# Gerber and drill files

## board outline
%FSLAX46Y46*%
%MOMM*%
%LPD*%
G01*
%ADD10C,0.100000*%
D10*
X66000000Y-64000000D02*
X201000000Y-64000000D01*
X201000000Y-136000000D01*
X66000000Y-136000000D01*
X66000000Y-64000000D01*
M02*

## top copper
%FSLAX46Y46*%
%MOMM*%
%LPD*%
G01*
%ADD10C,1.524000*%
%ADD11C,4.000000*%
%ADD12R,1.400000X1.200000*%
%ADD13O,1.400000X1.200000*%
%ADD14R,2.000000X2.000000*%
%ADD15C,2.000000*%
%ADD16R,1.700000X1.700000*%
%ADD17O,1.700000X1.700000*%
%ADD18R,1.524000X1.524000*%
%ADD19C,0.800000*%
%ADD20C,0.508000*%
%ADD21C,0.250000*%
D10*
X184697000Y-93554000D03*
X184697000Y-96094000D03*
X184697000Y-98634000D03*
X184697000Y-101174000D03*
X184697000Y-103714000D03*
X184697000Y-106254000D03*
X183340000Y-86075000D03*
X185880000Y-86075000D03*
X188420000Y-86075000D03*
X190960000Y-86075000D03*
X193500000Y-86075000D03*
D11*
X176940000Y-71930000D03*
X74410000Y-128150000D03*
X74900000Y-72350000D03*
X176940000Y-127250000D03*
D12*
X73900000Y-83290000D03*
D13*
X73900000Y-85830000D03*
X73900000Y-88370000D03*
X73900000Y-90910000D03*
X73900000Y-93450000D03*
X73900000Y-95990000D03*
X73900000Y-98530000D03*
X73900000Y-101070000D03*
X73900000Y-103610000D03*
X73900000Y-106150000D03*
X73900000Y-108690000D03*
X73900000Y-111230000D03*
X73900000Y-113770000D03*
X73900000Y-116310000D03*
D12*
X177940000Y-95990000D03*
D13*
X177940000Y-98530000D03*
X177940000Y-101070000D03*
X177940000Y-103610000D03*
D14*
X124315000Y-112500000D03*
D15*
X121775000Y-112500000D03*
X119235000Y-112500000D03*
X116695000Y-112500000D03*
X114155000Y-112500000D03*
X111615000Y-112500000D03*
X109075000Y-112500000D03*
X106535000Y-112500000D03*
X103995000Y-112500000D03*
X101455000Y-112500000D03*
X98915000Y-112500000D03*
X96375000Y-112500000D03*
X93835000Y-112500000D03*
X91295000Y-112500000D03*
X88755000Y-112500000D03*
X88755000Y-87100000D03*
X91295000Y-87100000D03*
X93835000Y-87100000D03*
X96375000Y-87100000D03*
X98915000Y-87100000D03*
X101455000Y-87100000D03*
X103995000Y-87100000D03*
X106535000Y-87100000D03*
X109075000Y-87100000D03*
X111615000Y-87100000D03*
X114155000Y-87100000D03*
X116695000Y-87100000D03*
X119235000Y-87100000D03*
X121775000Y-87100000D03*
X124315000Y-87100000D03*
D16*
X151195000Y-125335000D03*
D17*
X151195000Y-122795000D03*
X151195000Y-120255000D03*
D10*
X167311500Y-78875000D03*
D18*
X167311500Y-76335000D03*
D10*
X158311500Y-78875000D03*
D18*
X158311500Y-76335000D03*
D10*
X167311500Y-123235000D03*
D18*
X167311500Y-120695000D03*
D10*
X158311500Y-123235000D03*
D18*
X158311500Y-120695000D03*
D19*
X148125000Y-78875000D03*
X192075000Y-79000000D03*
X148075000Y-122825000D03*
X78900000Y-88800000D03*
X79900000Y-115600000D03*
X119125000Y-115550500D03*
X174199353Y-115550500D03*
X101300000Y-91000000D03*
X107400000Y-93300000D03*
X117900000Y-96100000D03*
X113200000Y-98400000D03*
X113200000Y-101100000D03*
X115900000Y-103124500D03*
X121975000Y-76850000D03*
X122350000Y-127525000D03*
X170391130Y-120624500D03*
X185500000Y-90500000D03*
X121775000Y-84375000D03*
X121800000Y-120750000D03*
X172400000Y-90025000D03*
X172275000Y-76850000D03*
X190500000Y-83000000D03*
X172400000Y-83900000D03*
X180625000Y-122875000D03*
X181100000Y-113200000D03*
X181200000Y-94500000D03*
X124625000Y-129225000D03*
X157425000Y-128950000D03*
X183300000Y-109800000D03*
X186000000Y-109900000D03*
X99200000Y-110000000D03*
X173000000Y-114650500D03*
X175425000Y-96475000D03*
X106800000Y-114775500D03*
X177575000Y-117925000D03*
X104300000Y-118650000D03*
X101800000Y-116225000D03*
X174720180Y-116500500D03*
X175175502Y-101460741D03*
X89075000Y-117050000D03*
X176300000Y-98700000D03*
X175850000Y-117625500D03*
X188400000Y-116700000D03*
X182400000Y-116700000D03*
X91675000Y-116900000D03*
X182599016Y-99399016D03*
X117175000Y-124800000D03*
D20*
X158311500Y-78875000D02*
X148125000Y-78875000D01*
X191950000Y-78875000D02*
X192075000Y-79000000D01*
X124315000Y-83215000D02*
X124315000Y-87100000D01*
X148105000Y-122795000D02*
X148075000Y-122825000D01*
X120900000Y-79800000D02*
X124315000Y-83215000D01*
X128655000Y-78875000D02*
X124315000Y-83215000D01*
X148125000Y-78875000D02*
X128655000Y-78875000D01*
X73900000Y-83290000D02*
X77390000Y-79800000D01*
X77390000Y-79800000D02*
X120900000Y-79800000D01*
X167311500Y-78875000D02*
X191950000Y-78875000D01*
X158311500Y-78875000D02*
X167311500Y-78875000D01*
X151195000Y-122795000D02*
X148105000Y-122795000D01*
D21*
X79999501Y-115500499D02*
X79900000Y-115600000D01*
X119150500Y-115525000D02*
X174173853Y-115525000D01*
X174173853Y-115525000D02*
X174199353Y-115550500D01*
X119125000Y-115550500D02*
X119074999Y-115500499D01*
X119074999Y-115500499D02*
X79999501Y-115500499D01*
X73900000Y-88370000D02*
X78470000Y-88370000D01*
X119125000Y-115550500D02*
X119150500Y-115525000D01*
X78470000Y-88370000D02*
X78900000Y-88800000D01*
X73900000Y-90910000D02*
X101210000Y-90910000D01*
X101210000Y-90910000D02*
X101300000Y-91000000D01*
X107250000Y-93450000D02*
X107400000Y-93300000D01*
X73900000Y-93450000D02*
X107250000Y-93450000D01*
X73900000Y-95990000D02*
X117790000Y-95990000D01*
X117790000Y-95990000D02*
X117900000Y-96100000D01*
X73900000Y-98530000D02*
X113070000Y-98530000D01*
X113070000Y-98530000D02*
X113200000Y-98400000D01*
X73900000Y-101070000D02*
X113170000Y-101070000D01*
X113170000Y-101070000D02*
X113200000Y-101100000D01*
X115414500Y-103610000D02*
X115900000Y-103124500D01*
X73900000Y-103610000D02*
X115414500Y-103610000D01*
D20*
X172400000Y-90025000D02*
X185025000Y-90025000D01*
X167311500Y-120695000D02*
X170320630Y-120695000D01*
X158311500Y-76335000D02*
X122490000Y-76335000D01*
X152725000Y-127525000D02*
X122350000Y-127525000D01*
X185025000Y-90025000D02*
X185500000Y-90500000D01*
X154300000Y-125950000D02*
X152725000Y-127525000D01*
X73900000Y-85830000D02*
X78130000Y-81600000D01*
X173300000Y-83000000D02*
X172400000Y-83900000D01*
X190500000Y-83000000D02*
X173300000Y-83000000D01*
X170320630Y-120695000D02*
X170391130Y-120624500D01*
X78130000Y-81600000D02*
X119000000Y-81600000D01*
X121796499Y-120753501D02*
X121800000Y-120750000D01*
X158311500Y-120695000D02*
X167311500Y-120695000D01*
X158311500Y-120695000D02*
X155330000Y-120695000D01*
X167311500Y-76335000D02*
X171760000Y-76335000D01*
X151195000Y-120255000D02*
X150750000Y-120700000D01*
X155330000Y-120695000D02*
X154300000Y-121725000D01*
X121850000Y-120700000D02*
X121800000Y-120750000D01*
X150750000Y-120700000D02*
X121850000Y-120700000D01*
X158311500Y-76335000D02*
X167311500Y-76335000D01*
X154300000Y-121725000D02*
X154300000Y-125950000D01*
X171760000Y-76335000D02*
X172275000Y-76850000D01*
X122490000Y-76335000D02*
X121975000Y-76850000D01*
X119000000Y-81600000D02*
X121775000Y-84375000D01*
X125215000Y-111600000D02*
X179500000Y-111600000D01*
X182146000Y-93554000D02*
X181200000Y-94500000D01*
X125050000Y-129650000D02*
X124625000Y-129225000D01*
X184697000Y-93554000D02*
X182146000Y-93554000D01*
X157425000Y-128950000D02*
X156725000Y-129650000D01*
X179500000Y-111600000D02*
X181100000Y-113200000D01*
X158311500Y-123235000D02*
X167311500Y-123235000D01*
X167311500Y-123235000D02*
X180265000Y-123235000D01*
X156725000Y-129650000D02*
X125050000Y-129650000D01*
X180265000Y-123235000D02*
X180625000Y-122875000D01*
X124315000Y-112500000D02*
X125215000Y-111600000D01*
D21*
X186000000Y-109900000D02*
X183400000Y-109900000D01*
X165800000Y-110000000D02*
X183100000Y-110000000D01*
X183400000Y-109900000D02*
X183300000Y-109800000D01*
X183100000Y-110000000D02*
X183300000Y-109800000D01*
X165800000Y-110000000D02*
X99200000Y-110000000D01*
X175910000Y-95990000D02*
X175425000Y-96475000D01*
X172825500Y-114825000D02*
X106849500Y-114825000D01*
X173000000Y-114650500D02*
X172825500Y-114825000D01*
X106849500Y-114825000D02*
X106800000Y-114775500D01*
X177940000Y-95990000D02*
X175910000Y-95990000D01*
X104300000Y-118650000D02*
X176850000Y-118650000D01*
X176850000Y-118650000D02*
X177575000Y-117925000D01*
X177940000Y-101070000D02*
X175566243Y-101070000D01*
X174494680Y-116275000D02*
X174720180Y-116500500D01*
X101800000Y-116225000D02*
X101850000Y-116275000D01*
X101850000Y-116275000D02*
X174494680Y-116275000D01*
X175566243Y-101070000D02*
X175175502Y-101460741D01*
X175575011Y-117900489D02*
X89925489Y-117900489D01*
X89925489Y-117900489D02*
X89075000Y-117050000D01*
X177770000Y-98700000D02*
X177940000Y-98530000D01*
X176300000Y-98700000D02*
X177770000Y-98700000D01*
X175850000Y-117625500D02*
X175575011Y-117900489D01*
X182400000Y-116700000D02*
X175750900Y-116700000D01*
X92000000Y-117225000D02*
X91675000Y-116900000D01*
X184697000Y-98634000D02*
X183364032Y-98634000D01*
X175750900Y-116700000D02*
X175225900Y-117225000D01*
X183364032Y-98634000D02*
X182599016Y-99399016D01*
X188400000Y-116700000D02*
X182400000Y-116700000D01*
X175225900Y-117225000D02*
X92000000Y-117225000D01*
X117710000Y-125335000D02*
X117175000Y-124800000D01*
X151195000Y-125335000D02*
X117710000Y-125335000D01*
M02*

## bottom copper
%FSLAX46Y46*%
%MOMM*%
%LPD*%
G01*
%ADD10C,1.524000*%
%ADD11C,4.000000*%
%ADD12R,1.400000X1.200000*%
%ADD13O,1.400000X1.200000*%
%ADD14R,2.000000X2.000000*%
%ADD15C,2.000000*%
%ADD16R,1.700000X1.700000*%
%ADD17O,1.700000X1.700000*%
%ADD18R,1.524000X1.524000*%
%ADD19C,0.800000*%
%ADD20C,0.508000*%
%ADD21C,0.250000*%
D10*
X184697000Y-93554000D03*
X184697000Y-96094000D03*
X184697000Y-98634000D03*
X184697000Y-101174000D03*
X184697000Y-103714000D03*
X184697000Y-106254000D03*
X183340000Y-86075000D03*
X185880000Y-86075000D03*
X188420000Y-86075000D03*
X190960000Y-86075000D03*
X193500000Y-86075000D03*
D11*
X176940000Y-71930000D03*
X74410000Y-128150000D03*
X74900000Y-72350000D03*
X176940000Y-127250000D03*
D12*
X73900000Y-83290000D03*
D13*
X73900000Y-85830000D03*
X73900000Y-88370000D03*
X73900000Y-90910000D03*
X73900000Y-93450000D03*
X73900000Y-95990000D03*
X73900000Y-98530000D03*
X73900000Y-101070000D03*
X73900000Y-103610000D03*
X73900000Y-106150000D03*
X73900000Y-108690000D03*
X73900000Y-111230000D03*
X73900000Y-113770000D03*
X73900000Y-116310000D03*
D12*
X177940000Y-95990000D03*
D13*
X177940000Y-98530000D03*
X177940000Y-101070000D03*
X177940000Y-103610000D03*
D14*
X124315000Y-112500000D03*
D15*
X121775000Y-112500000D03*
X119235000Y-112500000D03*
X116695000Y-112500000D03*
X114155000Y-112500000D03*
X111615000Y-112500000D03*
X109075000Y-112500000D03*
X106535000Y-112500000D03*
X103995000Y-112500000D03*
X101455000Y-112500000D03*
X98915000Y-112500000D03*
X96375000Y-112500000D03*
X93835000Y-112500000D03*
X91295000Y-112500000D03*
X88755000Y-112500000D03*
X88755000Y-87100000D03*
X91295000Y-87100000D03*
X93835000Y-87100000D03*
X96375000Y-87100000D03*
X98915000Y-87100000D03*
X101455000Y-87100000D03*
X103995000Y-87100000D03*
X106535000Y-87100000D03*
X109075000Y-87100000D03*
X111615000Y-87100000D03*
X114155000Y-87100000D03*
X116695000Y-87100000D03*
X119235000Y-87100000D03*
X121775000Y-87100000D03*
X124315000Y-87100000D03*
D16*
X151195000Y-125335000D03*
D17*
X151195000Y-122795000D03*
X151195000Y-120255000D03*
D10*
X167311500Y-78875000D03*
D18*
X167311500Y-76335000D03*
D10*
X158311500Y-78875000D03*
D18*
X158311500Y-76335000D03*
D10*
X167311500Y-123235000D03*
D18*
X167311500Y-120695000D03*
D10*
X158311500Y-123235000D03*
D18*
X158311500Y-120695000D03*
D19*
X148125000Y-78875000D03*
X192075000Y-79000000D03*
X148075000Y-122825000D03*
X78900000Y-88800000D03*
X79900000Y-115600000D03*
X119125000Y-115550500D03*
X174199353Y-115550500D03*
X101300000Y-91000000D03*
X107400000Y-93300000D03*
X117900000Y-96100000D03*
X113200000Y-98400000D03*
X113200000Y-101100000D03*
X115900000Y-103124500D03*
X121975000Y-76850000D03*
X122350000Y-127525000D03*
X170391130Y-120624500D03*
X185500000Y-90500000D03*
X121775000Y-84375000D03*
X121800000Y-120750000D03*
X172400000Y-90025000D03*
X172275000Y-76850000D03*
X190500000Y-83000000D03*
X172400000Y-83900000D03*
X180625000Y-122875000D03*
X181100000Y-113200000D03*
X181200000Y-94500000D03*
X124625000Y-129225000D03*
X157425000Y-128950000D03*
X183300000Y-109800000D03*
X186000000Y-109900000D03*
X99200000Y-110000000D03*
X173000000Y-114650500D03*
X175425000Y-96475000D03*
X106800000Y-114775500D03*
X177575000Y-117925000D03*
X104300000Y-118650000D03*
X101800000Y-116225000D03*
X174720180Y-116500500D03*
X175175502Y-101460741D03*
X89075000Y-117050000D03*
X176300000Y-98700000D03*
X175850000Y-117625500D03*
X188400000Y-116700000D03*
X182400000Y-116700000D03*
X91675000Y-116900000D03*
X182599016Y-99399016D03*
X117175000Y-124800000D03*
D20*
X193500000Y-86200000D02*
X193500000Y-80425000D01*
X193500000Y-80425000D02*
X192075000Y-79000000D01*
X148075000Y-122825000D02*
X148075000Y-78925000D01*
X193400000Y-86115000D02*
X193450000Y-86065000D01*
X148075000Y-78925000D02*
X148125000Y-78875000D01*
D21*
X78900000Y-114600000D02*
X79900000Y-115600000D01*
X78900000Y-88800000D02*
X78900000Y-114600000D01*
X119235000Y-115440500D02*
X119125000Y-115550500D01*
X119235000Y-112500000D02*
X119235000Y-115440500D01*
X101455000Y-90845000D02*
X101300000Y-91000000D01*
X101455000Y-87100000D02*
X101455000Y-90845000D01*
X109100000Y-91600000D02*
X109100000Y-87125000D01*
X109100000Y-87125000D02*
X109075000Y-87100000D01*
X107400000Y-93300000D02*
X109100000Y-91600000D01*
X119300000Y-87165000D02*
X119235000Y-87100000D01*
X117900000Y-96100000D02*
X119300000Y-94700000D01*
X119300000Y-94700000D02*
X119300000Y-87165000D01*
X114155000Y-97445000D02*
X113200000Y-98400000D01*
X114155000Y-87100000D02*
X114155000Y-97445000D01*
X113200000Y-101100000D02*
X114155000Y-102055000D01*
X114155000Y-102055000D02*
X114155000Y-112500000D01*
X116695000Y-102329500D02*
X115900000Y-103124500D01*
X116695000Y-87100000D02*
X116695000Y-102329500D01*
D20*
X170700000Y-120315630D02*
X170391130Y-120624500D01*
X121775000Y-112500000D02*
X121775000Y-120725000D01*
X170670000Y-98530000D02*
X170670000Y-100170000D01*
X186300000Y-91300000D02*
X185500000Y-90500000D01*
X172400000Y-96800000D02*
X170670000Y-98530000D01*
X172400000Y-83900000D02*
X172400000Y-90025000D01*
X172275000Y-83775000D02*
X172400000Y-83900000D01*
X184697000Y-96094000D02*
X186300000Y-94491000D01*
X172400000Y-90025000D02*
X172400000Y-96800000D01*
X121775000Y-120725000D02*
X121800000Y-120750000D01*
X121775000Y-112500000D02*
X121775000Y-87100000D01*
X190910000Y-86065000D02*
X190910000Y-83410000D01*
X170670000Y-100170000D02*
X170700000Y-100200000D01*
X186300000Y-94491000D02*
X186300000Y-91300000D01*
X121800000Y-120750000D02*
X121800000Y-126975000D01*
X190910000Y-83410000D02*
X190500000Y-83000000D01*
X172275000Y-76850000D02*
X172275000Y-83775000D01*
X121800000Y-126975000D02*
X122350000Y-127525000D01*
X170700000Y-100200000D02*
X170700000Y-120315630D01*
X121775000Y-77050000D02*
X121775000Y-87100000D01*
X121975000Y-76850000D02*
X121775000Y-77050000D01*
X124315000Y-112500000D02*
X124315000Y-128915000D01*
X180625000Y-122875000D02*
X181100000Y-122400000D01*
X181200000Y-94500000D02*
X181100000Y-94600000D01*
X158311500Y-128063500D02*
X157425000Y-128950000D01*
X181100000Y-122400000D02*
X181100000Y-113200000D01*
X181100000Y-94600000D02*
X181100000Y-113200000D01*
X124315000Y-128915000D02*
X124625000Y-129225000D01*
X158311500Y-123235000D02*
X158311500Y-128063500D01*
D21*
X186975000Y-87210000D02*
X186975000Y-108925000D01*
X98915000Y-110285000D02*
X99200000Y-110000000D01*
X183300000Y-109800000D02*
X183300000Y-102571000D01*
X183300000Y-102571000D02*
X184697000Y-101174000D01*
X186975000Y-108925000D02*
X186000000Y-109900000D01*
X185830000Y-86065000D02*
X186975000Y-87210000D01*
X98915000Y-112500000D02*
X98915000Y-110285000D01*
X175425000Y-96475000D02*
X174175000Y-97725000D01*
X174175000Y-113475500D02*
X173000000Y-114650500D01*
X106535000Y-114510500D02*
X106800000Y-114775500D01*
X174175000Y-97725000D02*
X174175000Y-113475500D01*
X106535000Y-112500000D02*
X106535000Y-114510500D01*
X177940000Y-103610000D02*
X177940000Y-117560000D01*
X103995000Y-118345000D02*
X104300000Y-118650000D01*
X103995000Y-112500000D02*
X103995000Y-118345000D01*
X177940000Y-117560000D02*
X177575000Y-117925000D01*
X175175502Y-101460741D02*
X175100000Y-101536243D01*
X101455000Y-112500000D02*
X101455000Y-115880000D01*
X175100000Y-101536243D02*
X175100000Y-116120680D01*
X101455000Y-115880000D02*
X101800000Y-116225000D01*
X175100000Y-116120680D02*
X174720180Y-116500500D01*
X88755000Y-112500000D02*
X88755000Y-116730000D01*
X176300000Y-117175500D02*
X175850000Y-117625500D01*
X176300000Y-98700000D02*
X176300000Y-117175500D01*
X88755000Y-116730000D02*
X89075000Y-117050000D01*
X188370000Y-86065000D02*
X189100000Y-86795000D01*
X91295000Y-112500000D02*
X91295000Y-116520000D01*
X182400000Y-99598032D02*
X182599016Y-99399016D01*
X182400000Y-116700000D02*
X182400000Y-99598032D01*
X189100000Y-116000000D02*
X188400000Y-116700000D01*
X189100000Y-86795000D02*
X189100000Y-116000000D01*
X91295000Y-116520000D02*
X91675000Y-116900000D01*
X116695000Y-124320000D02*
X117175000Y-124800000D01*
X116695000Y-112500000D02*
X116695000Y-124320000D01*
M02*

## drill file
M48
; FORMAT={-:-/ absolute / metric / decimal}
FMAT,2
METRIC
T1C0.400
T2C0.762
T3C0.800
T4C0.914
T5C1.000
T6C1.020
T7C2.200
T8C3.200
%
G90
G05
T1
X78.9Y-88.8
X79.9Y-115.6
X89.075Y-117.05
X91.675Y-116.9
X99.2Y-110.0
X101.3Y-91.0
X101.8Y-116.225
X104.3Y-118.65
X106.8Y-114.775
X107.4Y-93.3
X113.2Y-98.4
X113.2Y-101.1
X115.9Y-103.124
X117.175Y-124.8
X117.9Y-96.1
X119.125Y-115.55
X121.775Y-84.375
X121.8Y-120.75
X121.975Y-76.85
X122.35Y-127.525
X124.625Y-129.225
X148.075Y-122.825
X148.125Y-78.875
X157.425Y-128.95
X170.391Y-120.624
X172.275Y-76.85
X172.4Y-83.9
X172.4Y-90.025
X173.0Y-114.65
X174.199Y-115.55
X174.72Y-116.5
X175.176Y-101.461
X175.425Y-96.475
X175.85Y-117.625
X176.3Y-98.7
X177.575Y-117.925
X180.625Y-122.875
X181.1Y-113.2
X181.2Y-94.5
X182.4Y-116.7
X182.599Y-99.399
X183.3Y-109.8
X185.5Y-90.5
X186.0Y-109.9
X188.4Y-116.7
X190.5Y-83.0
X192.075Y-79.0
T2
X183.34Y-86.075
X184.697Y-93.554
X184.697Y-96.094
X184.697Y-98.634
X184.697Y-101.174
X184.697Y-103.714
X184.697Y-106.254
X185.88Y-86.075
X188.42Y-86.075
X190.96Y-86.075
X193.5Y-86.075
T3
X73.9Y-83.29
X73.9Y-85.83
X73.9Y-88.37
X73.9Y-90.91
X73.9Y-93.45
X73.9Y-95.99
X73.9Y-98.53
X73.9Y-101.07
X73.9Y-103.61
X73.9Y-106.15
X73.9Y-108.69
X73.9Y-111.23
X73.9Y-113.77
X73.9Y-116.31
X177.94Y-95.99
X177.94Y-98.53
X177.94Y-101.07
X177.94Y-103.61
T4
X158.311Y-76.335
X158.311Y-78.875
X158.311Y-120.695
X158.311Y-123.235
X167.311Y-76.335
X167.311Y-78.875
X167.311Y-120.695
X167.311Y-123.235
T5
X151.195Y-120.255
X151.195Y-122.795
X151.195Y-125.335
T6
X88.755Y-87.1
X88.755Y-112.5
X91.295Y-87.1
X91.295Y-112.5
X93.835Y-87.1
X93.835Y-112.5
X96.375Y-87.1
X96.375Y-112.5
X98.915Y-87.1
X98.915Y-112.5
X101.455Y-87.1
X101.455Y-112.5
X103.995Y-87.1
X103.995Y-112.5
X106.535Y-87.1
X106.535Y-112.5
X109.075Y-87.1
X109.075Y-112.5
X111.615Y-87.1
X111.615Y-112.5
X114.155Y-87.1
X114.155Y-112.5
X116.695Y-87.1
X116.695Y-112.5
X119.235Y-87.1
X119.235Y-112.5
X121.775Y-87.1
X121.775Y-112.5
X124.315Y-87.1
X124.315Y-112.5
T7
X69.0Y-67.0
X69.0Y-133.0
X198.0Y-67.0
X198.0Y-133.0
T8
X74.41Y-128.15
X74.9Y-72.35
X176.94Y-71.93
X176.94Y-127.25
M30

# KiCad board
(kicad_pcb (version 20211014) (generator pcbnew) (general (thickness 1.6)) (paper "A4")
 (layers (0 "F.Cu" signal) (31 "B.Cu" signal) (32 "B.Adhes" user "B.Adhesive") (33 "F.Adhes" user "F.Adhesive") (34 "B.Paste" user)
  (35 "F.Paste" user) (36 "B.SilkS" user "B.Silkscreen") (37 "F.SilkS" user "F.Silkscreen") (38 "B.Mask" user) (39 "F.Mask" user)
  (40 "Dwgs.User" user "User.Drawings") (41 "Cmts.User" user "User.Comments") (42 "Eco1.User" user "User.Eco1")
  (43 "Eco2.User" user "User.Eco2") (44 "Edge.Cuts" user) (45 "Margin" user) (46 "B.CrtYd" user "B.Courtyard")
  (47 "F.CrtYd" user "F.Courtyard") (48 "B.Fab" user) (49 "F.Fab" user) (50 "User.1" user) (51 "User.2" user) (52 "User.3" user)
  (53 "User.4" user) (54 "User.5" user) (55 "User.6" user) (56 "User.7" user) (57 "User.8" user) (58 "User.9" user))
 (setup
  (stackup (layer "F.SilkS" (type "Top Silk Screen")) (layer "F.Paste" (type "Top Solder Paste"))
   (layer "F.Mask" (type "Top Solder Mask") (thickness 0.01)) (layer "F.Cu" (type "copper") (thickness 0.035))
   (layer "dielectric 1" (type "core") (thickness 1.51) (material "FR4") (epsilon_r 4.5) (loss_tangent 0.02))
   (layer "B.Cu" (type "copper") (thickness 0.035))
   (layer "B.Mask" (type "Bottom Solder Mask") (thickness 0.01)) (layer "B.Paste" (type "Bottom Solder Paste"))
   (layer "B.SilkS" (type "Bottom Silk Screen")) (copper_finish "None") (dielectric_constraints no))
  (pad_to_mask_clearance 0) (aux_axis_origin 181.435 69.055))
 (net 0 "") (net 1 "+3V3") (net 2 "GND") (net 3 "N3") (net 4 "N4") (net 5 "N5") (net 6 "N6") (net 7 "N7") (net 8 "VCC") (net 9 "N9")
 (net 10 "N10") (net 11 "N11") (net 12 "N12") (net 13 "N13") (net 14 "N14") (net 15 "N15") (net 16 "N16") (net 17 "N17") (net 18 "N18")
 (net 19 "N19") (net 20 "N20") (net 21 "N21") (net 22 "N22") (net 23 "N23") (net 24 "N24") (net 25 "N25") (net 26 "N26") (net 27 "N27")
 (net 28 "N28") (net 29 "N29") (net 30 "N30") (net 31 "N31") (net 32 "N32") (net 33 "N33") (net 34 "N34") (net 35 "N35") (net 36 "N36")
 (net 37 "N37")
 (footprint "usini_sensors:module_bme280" (layer "F.Cu") (at 189.777 106)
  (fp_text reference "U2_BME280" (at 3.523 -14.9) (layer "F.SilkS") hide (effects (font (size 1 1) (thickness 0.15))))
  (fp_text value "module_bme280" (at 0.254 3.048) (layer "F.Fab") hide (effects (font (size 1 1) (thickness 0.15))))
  (pad "1" thru_hole circle locked (at -5.08 -12.446) (size 1.524 1.524) (drill 0.762) (layers *.Cu *.Mask) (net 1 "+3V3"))
  (pad "2" thru_hole circle locked (at -5.08 -9.906) (size 1.524 1.524) (drill 0.762) (layers *.Cu *.Mask) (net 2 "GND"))
  (pad "3" thru_hole circle locked (at -5.08 -7.366) (size 1.524 1.524) (drill 0.762) (layers *.Cu *.Mask) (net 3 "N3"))
  (pad "4" thru_hole circle locked (at -5.08 -4.826) (size 1.524 1.524) (drill 0.762) (layers *.Cu *.Mask) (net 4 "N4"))
  (pad "5" thru_hole circle locked (at -5.08 -2.286) (size 1.524 1.524) (drill 0.762) (layers *.Cu *.Mask) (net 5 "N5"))
  (pad "6" thru_hole circle locked (at -5.08 0.254) (size 1.524 1.524) (drill 0.762) (layers *.Cu *.Mask) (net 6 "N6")))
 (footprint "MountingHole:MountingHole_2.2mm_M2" (layer "F.Cu") (at 69 67)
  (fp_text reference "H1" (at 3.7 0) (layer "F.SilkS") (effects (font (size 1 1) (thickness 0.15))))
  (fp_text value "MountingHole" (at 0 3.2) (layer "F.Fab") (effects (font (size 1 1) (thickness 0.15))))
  (pad "" np_thru_hole circle locked (at 0 0) (size 2.2 2.2) (drill 2.2) (layers *.Cu *.Mask)))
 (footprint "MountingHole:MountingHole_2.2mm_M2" (layer "F.Cu") (at 198 67)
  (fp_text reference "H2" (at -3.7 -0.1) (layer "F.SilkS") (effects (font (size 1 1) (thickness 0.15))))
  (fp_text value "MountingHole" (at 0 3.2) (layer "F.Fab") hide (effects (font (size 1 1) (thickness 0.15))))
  (pad "" np_thru_hole circle locked (at 0 0) (size 2.2 2.2) (drill 2.2) (layers *.Cu *.Mask)))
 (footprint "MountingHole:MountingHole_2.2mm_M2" (layer "F.Cu") (at 198 133)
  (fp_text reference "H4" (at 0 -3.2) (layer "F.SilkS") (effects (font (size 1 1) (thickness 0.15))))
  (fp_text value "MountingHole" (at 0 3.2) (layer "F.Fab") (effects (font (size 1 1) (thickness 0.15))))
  (pad "" np_thru_hole circle locked (at 0 0) (size 2.2 2.2) (drill 2.2) (layers *.Cu *.Mask)))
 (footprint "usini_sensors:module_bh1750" (layer "F.Cu") (at 193.5 86.075 90)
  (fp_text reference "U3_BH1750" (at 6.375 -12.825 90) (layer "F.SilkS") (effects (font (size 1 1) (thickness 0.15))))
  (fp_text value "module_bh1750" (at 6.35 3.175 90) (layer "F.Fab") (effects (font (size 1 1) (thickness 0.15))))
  (pad "1" thru_hole circle locked (at 0 -10.16 90) (size 1.524 1.524) (drill 0.762) (layers *.Cu *.Mask) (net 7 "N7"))
  (pad "2" thru_hole circle locked (at 0 -7.62 90) (size 1.524 1.524) (drill 0.762) (layers *.Cu *.Mask) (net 4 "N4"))
  (pad "3" thru_hole circle locked (at 0 -5.08 90) (size 1.524 1.524) (drill 0.762) (layers *.Cu *.Mask) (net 3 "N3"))
  (pad "4" thru_hole circle locked (at 0 -2.54 90) (size 1.524 1.524) (drill 0.762) (layers *.Cu *.Mask) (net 2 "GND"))
  (pad "5" thru_hole circle locked (at 0 0 90) (size 1.524 1.524) (drill 0.762) (layers *.Cu *.Mask) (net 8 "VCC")))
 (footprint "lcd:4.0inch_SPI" (layer "F.Cu") (at 71.9 68.93)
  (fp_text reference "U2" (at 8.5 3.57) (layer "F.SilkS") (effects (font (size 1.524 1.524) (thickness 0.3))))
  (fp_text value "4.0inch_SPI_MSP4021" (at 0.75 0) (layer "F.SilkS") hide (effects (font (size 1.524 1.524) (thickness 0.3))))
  (pad "" np_thru_hole circle (at 105.04 3 270) (size 4 4) (drill 3.2) (layers F&B.Cu *.Mask))
  (pad "" np_thru_hole circle (at 2.51 59.22 270) (size 4 4) (drill 3.2) (layers F&B.Cu *.Mask))
  (pad "" np_thru_hole circle (at 3 3.42 270) (size 4 4) (drill 3.2) (layers F&B.Cu *.Mask))
  (pad "" np_thru_hole circle (at 105.04 58.32 270) (size 4 4) (drill 3.2) (layers F&B.Cu *.Mask))
  (pad "1" thru_hole rect (at 2 14.36 270) (size 1.2 1.4) (drill 0.8) (layers *.Cu *.Mask) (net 8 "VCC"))
  (pad "2" thru_hole oval (at 2 16.9 270) (size 1.2 1.4) (drill 0.8) (layers *.Cu *.Mask) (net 2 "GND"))
  (pad "3" thru_hole oval (at 2 19.44 270) (size 1.2 1.4) (drill 0.8) (layers *.Cu *.Mask) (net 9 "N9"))
  (pad "4" thru_hole oval (at 2 21.98 270) (size 1.2 1.4) (drill 0.8) (layers *.Cu *.Mask) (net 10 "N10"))
  (pad "5" thru_hole oval (at 2 24.52 270) (size 1.2 1.4) (drill 0.8) (layers *.Cu *.Mask) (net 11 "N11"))
  (pad "6" thru_hole oval (at 2 27.06 270) (size 1.2 1.4) (drill 0.8) (layers *.Cu *.Mask) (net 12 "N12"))
  (pad "7" thru_hole oval (at 2 29.6 270) (size 1.2 1.4) (drill 0.8) (layers *.Cu *.Mask) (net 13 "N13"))
  (pad "8" thru_hole oval (at 2 32.14 270) (size 1.2 1.4) (drill 0.8) (layers *.Cu *.Mask) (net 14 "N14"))
  (pad "9" thru_hole oval (at 2 34.68 270) (size 1.2 1.4) (drill 0.8) (layers *.Cu *.Mask) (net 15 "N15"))
  (pad "10" thru_hole oval (at 2 37.22 270) (size 1.2 1.4) (drill 0.8) (layers *.Cu *.Mask) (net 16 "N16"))
  (pad "11" thru_hole oval (at 2 39.76 270) (size 1.2 1.4) (drill 0.8) (layers *.Cu *.Mask) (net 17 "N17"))
  (pad "12" thru_hole oval (at 2 42.3 270) (size 1.2 1.4) (drill 0.8) (layers *.Cu *.Mask) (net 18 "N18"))
  (pad "13" thru_hole oval (at 2 44.84 270) (size 1.2 1.4) (drill 0.8) (layers *.Cu *.Mask) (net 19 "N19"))
  (pad "14" thru_hole oval (at 2 47.38 270) (size 1.2 1.4) (drill 0.8) (layers *.Cu *.Mask) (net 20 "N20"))
  (pad "15" thru_hole rect (at 106.04 27.06 270) (size 1.2 1.4) (drill 0.8) (layers *.Cu *.Mask) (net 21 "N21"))
  (pad "16" thru_hole oval (at 106.04 29.6 270) (size 1.2 1.4) (drill 0.8) (layers *.Cu *.Mask) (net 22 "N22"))
  (pad "17" thru_hole oval (at 106.04 32.14 270) (size 1.2 1.4) (drill 0.8) (layers *.Cu *.Mask) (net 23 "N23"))
  (pad "18" thru_hole oval (at 106.04 34.68 270) (size 1.2 1.4) (drill 0.8) (layers *.Cu *.Mask) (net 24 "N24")))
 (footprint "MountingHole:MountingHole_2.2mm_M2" (layer "F.Cu") (at 69 133)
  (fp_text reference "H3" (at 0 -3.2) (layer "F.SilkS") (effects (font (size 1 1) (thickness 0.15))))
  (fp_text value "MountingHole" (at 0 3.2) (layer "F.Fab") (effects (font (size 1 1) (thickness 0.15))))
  (pad "" np_thru_hole circle locked (at 0 0) (size 2.2 2.2) (drill 2.2) (layers *.Cu *.Mask)))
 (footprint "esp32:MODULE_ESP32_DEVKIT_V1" (layer "B.Cu") (at 108.8 99.8 90)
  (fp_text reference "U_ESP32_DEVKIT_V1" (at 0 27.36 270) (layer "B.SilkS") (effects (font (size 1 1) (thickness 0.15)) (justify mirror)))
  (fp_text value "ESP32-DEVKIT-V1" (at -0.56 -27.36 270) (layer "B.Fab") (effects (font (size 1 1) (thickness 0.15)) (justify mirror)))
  (pad "1" thru_hole rect (at -12.7 15.515 90) (size 2 2) (drill 1.02) (layers *.Cu *.Mask) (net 1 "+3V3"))
  (pad "2" thru_hole circle (at -12.7 12.975 90) (size 2 2) (drill 1.02) (layers *.Cu *.Mask) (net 2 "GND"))
  (pad "3" thru_hole circle (at -12.7 10.435 90) (size 2 2) (drill 1.02) (layers *.Cu *.Mask) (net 9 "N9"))
  (pad "4" thru_hole circle (at -12.7 7.895 90) (size 2 2) (drill 1.02) (layers *.Cu *.Mask) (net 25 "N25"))
  (pad "5" thru_hole circle (at -12.7 5.355 90) (size 2 2) (drill 1.02) (layers *.Cu *.Mask) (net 14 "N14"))
  (pad "6" thru_hole circle (at -12.7 2.815 90) (size 2 2) (drill 1.02) (layers *.Cu *.Mask) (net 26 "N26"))
  (pad "7" thru_hole circle (at -12.7 0.275 90) (size 2 2) (drill 1.02) (layers *.Cu *.Mask) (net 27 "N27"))
  (pad "8" thru_hole circle (at -12.7 -2.265 90) (size 2 2) (drill 1.02) (layers *.Cu *.Mask) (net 21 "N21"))
  (pad "9" thru_hole circle (at -12.7 -4.805 90) (size 2 2) (drill 1.02) (layers *.Cu *.Mask) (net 24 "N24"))
  (pad "10" thru_hole circle (at -12.7 -7.345 90) (size 2 2) (drill 1.02) (layers *.Cu *.Mask) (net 23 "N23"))
  (pad "11" thru_hole circle (at -12.7 -9.885 90) (size 2 2) (drill 1.02) (layers *.Cu *.Mask) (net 4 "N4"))
  (pad "12" thru_hole circle (at -12.7 -12.425 90) (size 2 2) (drill 1.02) (layers *.Cu *.Mask) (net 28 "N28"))
  (pad "13" thru_hole circle (at -12.7 -14.965 90) (size 2 2) (drill 1.02) (layers *.Cu *.Mask) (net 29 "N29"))
  (pad "14" thru_hole circle (at -12.7 -17.505 90) (size 2 2) (drill 1.02) (layers *.Cu *.Mask) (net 3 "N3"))
  (pad "15" thru_hole circle (at -12.7 -20.045 90) (size 2 2) (drill 1.02) (layers *.Cu *.Mask) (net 22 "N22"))
  (pad "16" thru_hole circle (at 12.7 -20.045 90) (size 2 2) (drill 1.02) (layers *.Cu *.Mask) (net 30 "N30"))
  (pad "17" thru_hole circle (at 12.7 -17.505 90) (size 2 2) (drill 1.02) (layers *.Cu *.Mask) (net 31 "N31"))
  (pad "18" thru_hole circle (at 12.7 -14.965 90) (size 2 2) (drill 1.02) (layers *.Cu *.Mask) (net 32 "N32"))
  (pad "19" thru_hole circle (at 12.7 -12.425 90) (size 2 2) (drill 1.02) (layers *.Cu *.Mask) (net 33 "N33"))
  (pad "20" thru_hole circle (at 12.7 -9.885 90) (size 2 2) (drill 1.02) (layers *.Cu *.Mask) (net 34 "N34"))
  (pad "21" thru_hole circle (at 12.7 -7.345 90) (size 2 2) (drill 1.02) (layers *.Cu *.Mask) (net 10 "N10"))
  (pad "22" thru_hole circle (at 12.7 -4.805 90) (size 2 2) (drill 1.02) (layers *.Cu *.Mask) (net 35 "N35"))
  (pad "23" thru_hole circle (at 12.7 -2.265 90) (size 2 2) (drill 1.02) (layers *.Cu *.Mask) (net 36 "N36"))
  (pad "24" thru_hole circle (at 12.7 0.275 90) (size 2 2) (drill 1.02) (layers *.Cu *.Mask) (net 11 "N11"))
  (pad "25" thru_hole circle (at 12.7 2.815 90) (size 2 2) (drill 1.02) (layers *.Cu *.Mask) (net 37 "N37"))
  (pad "26" thru_hole circle (at 12.7 5.355 90) (size 2 2) (drill 1.02) (layers *.Cu *.Mask) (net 13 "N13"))
  (pad "27" thru_hole circle (at 12.7 7.895 90) (size 2 2) (drill 1.02) (layers *.Cu *.Mask) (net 15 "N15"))
  (pad "28" thru_hole circle (at 12.7 10.435 90) (size 2 2) (drill 1.02) (layers *.Cu *.Mask) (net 12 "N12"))
  (pad "29" thru_hole circle (at 12.7 12.975 90) (size 2 2) (drill 1.02) (layers *.Cu *.Mask) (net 2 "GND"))
  (pad "30" thru_hole circle (at 12.7 15.515 90) (size 2 2) (drill 1.02) (layers *.Cu *.Mask) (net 8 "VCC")))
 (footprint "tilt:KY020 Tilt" (layer "B.Cu") (at 135.195 115.745 -90)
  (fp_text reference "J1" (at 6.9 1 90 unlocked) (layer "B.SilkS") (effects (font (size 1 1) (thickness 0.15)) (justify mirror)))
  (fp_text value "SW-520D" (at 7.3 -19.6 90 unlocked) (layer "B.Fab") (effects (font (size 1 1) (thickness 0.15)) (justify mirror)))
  (pad "1" thru_hole rect (at 9.59 -16) (size 1.7 1.7) (drill 1) (layers *.Cu *.Mask) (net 25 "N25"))
  (pad "2" thru_hole oval (at 7.05 -16) (size 1.7 1.7) (drill 1) (layers *.Cu *.Mask) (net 8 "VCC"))
  (pad "3" thru_hole oval (at 4.51 -16) (size 1.7 1.7) (drill 1) (layers *.Cu *.Mask) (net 2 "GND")))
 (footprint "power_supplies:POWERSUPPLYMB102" (layer "B.Cu") (at 154.3115 126.235 90)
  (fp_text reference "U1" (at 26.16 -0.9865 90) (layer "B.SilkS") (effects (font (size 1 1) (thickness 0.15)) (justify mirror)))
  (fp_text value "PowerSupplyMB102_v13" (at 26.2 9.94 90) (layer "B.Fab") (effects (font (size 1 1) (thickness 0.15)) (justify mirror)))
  (pad "1" thru_hole circle (at 47.36 13 90) (size 1.524 1.524) (drill 0.9144) (layers *.Cu *.Mask) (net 8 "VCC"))
  (pad "2" thru_hole rect (at 49.9 13 90) (size 1.524 1.524) (drill 0.9144) (layers *.Cu *.Mask) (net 2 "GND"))
  (pad "3" thru_hole circle (at 47.36 4 90) (size 1.524 1.524) (drill 0.9144) (layers *.Cu *.Mask) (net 8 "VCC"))
  (pad "4" thru_hole rect (at 49.9 4 90) (size 1.524 1.524) (drill 0.9144) (layers *.Cu *.Mask) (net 2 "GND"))
  (pad "5" thru_hole circle (at 3 13 90) (size 1.524 1.524) (drill 0.9144) (layers *.Cu *.Mask) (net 1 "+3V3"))
  (pad "6" thru_hole rect (at 5.54 13 90) (size 1.524 1.524) (drill 0.9144) (layers *.Cu *.Mask) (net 2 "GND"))
  (pad "7" thru_hole circle (at 3 4 90) (size 1.524 1.524) (drill 0.9144) (layers *.Cu *.Mask) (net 1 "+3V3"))
  (pad "8" thru_hole rect (at 5.54 4 90) (size 1.524 1.524) (drill 0.9144) (layers *.Cu *.Mask) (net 2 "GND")))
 (gr_rect (start 66 64) (end 201 136) (layer "Edge.Cuts") (width 0.1) (fill none))
 (segment (start 158.3115 78.875) (end 148.125 78.875) (width 0.508) (layer "F.Cu") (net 8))
 (segment (start 191.95 78.875) (end 192.075 79) (width 0.508) (layer "F.Cu") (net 8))
 (segment (start 124.315 83.215) (end 124.315 87.1) (width 0.508) (layer "F.Cu") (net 8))
 (segment (start 148.105 122.795) (end 148.075 122.825) (width 0.508) (layer "F.Cu") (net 8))
 (segment (start 120.9 79.8) (end 124.315 83.215) (width 0.508) (layer "F.Cu") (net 8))
 (segment (start 128.655 78.875) (end 124.315 83.215) (width 0.508) (layer "F.Cu") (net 8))
 (segment (start 148.125 78.875) (end 128.655 78.875) (width 0.508) (layer "F.Cu") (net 8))
 (segment (start 73.9 83.29) (end 77.39 79.8) (width 0.508) (layer "F.Cu") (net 8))
 (segment (start 77.39 79.8) (end 120.9 79.8) (width 0.508) (layer "F.Cu") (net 8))
 (segment (start 167.3115 78.875) (end 191.95 78.875) (width 0.508) (layer "F.Cu") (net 8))
 (segment (start 158.3115 78.875) (end 167.3115 78.875) (width 0.508) (layer "F.Cu") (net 8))
 (segment (start 151.195 122.795) (end 148.105 122.795) (width 0.508) (layer "F.Cu") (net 8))
 (via (at 148.125 78.875) (size 0.8) (drill 0.4) (layers "F.Cu" "B.Cu") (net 8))
 (via (at 192.075 79) (size 0.8) (drill 0.4) (layers "F.Cu" "B.Cu") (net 8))
 (via (at 148.075 122.825) (size 0.8) (drill 0.4) (layers "F.Cu" "B.Cu") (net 8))
 (segment (start 193.5 86.2) (end 193.5 80.425) (width 0.508) (layer "B.Cu") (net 8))
 (segment (start 193.5 80.425) (end 192.075 79) (width 0.508) (layer "B.Cu") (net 8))
 (segment (start 148.075 122.825) (end 148.075 78.925) (width 0.508) (layer "B.Cu") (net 8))
 (segment (start 193.4 86.115) (end 193.45 86.065) (width 0.508) (layer "B.Cu") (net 8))
 (segment (start 148.075 78.925) (end 148.125 78.875) (width 0.508) (layer "B.Cu") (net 8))
 (segment (start 79.999501 115.500499) (end 79.9 115.6) (width 0.25) (layer "F.Cu") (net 9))
 (segment (start 119.1505 115.525) (end 174.173853 115.525) (width 0.25) (layer "F.Cu") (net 9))
 (segment (start 174.173853 115.525) (end 174.199353 115.5505) (width 0.25) (layer "F.Cu") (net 9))
 (segment (start 119.125 115.5505) (end 119.074999 115.500499) (width 0.25) (layer "F.Cu") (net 9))
 (segment (start 119.074999 115.500499) (end 79.999501 115.500499) (width 0.25) (layer "F.Cu") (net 9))
 (segment (start 73.9 88.37) (end 78.47 88.37) (width 0.25) (layer "F.Cu") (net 9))
 (segment (start 119.125 115.5505) (end 119.1505 115.525) (width 0.25) (layer "F.Cu") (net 9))
 (segment (start 78.47 88.37) (end 78.9 88.8) (width 0.25) (layer "F.Cu") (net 9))
 (via (at 78.9 88.8) (size 0.8) (drill 0.4) (layers "F.Cu" "B.Cu") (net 9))
 (via (at 79.9 115.6) (size 0.8) (drill 0.4) (layers "F.Cu" "B.Cu") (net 9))
 (via (at 119.125 115.5505) (size 0.8) (drill 0.4) (layers "F.Cu" "B.Cu") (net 9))
 (via (at 174.199353 115.5505) (size 0.8) (drill 0.4) (layers "F.Cu" "B.Cu") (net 9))
 (segment (start 78.9 114.6) (end 79.9 115.6) (width 0.25) (layer "B.Cu") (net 9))
 (segment (start 78.9 88.8) (end 78.9 114.6) (width 0.25) (layer "B.Cu") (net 9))
 (segment (start 119.235 115.4405) (end 119.125 115.5505) (width 0.25) (layer "B.Cu") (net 9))
 (segment (start 119.235 112.5) (end 119.235 115.4405) (width 0.25) (layer "B.Cu") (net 9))
 (segment (start 73.9 90.91) (end 101.21 90.91) (width 0.25) (layer "F.Cu") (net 10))
 (segment (start 101.21 90.91) (end 101.3 91) (width 0.25) (layer "F.Cu") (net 10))
 (via (at 101.3 91) (size 0.8) (drill 0.4) (layers "F.Cu" "B.Cu") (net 10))
 (segment (start 101.455 90.845) (end 101.3 91) (width 0.25) (layer "B.Cu") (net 10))
 (segment (start 101.455 87.1) (end 101.455 90.845) (width 0.25) (layer "B.Cu") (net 10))
 (segment (start 107.25 93.45) (end 107.4 93.3) (width 0.25) (layer "F.Cu") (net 11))
 (segment (start 73.9 93.45) (end 107.25 93.45) (width 0.25) (layer "F.Cu") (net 11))
 (via (at 107.4 93.3) (size 0.8) (drill 0.4) (layers "F.Cu" "B.Cu") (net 11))
 (segment (start 109.1 91.6) (end 109.1 87.125) (width 0.25) (layer "B.Cu") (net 11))
 (segment (start 109.1 87.125) (end 109.075 87.1) (width 0.25) (layer "B.Cu") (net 11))
 (segment (start 107.4 93.3) (end 109.1 91.6) (width 0.25) (layer "B.Cu") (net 11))
 (segment (start 73.9 95.99) (end 117.79 95.99) (width 0.25) (layer "F.Cu") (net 12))
 (segment (start 117.79 95.99) (end 117.9 96.1) (width 0.25) (layer "F.Cu") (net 12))
 (via (at 117.9 96.1) (size 0.8) (drill 0.4) (layers "F.Cu" "B.Cu") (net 12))
 (segment (start 119.3 87.165) (end 119.235 87.1) (width 0.25) (layer "B.Cu") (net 12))
 (segment (start 117.9 96.1) (end 119.3 94.7) (width 0.25) (layer "B.Cu") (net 12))
 (segment (start 119.3 94.7) (end 119.3 87.165) (width 0.25) (layer "B.Cu") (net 12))
 (segment (start 73.9 98.53) (end 113.07 98.53) (width 0.25) (layer "F.Cu") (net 13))
 (segment (start 113.07 98.53) (end 113.2 98.4) (width 0.25) (layer "F.Cu") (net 13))
 (via (at 113.2 98.4) (size 0.8) (drill 0.4) (layers "F.Cu" "B.Cu") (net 13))
 (segment (start 114.155 97.445) (end 113.2 98.4) (width 0.25) (layer "B.Cu") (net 13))
 (segment (start 114.155 87.1) (end 114.155 97.445) (width 0.25) (layer "B.Cu") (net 13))
 (segment (start 73.9 101.07) (end 113.17 101.07) (width 0.25) (layer "F.Cu") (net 14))
 (segment (start 113.17 101.07) (end 113.2 101.1) (width 0.25) (layer "F.Cu") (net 14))
 (via (at 113.2 101.1) (size 0.8) (drill 0.4) (layers "F.Cu" "B.Cu") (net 14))
 (segment (start 113.2 101.1) (end 114.155 102.055) (width 0.25) (layer "B.Cu") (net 14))
 (segment (start 114.155 102.055) (end 114.155 112.5) (width 0.25) (layer "B.Cu") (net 14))
 (segment (start 115.4145 103.61) (end 115.9 103.1245) (width 0.25) (layer "F.Cu") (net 15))
 (segment (start 73.9 103.61) (end 115.4145 103.61) (width 0.25) (layer "F.Cu") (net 15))
 (via (at 115.9 103.1245) (size 0.8) (drill 0.4) (layers "F.Cu" "B.Cu") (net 15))
 (segment (start 116.695 102.3295) (end 115.9 103.1245) (width 0.25) (layer "B.Cu") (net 15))
 (segment (start 116.695 87.1) (end 116.695 102.3295) (width 0.25) (layer "B.Cu") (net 15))
 (segment (start 172.4 90.025) (end 185.025 90.025) (width 0.508) (layer "F.Cu") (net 2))
 (segment (start 167.3115 120.695) (end 170.32063 120.695) (width 0.508) (layer "F.Cu") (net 2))
 (segment (start 158.3115 76.335) (end 122.49 76.335) (width 0.508) (layer "F.Cu") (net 2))
 (segment (start 152.725 127.525) (end 122.35 127.525) (width 0.508) (layer "F.Cu") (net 2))
 (segment (start 185.025 90.025) (end 185.5 90.5) (width 0.508) (layer "F.Cu") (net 2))
 (segment (start 154.3 125.95) (end 152.725 127.525) (width 0.508) (layer "F.Cu") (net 2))
 (segment (start 73.9 85.83) (end 78.13 81.6) (width 0.508) (layer "F.Cu") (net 2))
 (segment (start 173.3 83) (end 172.4 83.9) (width 0.508) (layer "F.Cu") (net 2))
 (segment (start 190.5 83) (end 173.3 83) (width 0.508) (layer "F.Cu") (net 2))
 (segment (start 170.32063 120.695) (end 170.39113 120.6245) (width 0.508) (layer "F.Cu") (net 2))
 (segment (start 78.13 81.6) (end 119 81.6) (width 0.508) (layer "F.Cu") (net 2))
 (segment (start 121.796499 120.753501) (end 121.8 120.75) (width 0.508) (layer "F.Cu") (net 2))
 (segment (start 158.3115 120.695) (end 167.3115 120.695) (width 0.508) (layer "F.Cu") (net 2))
 (segment (start 158.3115 120.695) (end 155.33 120.695) (width 0.508) (layer "F.Cu") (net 2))
 (segment (start 167.3115 76.335) (end 171.76 76.335) (width 0.508) (layer "F.Cu") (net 2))
 (segment (start 151.195 120.255) (end 150.75 120.7) (width 0.508) (layer "F.Cu") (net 2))
 (segment (start 155.33 120.695) (end 154.3 121.725) (width 0.508) (layer "F.Cu") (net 2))
 (segment (start 121.85 120.7) (end 121.8 120.75) (width 0.508) (layer "F.Cu") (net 2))
 (segment (start 150.75 120.7) (end 121.85 120.7) (width 0.508) (layer "F.Cu") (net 2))
 (segment (start 158.3115 76.335) (end 167.3115 76.335) (width 0.508) (layer "F.Cu") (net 2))
 (segment (start 154.3 121.725) (end 154.3 125.95) (width 0.508) (layer "F.Cu") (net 2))
 (segment (start 171.76 76.335) (end 172.275 76.85) (width 0.508) (layer "F.Cu") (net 2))
 (segment (start 122.49 76.335) (end 121.975 76.85) (width 0.508) (layer "F.Cu") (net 2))
 (segment (start 119 81.6) (end 121.775 84.375) (width 0.508) (layer "F.Cu") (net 2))
 (via (at 121.975 76.85) (size 0.8) (drill 0.4) (layers "F.Cu" "B.Cu") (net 2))
 (via (at 122.35 127.525) (size 0.8) (drill 0.4) (layers "F.Cu" "B.Cu") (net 2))
 (via (at 170.39113 120.6245) (size 0.8) (drill 0.4) (layers "F.Cu" "B.Cu") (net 2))
 (via (at 185.5 90.5) (size 0.8) (drill 0.4) (layers "F.Cu" "B.Cu") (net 2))
 (via (at 121.775 84.375) (size 0.8) (drill 0.4) (layers "F.Cu" "B.Cu") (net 2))
 (via (at 121.8 120.75) (size 0.8) (drill 0.4) (layers "F.Cu" "B.Cu") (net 2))
 (via (at 172.4 90.025) (size 0.8) (drill 0.4) (layers "F.Cu" "B.Cu") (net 2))
 (via (at 172.275 76.85) (size 0.8) (drill 0.4) (layers "F.Cu" "B.Cu") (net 2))
 (via (at 190.5 83) (size 0.8) (drill 0.4) (layers "F.Cu" "B.Cu") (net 2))
 (via (at 172.4 83.9) (size 0.8) (drill 0.4) (layers "F.Cu" "B.Cu") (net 2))
 (segment (start 170.7 120.31563) (end 170.39113 120.6245) (width 0.508) (layer "B.Cu") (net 2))
 (segment (start 121.775 112.5) (end 121.775 120.725) (width 0.508) (layer "B.Cu") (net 2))
 (segment (start 170.67 98.53) (end 170.67 100.17) (width 0.508) (layer "B.Cu") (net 2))
 (segment (start 186.3 91.3) (end 185.5 90.5) (width 0.508) (layer "B.Cu") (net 2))
 (segment (start 172.4 96.8) (end 170.67 98.53) (width 0.508) (layer "B.Cu") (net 2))
 (segment (start 172.4 83.9) (end 172.4 90.025) (width 0.508) (layer "B.Cu") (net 2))
 (segment (start 172.275 83.775) (end 172.4 83.9) (width 0.508) (layer "B.Cu") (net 2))
 (segment (start 184.697 96.094) (end 186.3 94.491) (width 0.508) (layer "B.Cu") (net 2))
 (segment (start 172.4 90.025) (end 172.4 96.8) (width 0.508) (layer "B.Cu") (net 2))
 (segment (start 121.775 120.725) (end 121.8 120.75) (width 0.508) (layer "B.Cu") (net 2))
 (segment (start 121.775 112.5) (end 121.775 87.1) (width 0.508) (layer "B.Cu") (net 2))
 (segment (start 190.91 86.065) (end 190.91 83.41) (width 0.508) (layer "B.Cu") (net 2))
 (segment (start 170.67 100.17) (end 170.7 100.2) (width 0.508) (layer "B.Cu") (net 2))
 (segment (start 186.3 94.491) (end 186.3 91.3) (width 0.508) (layer "B.Cu") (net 2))
 (segment (start 121.8 120.75) (end 121.8 126.975) (width 0.508) (layer "B.Cu") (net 2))
 (segment (start 190.91 83.41) (end 190.5 83) (width 0.508) (layer "B.Cu") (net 2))
 (segment (start 172.275 76.85) (end 172.275 83.775) (width 0.508) (layer "B.Cu") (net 2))
 (segment (start 121.8 126.975) (end 122.35 127.525) (width 0.508) (layer "B.Cu") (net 2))
 (segment (start 170.7 100.2) (end 170.7 120.31563) (width 0.508) (layer "B.Cu") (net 2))
 (segment (start 121.775 77.05) (end 121.775 87.1) (width 0.508) (layer "B.Cu") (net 2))
 (segment (start 121.975 76.85) (end 121.775 77.05) (width 0.508) (layer "B.Cu") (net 2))
 (segment (start 125.215 111.6) (end 179.5 111.6) (width 0.508) (layer "F.Cu") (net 1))
 (segment (start 182.146 93.554) (end 181.2 94.5) (width 0.508) (layer "F.Cu") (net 1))
 (segment (start 125.05 129.65) (end 124.625 129.225) (width 0.508) (layer "F.Cu") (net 1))
 (segment (start 184.697 93.554) (end 182.146 93.554) (width 0.508) (layer "F.Cu") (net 1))
 (segment (start 157.425 128.95) (end 156.725 129.65) (width 0.508) (layer "F.Cu") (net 1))
 (segment (start 179.5 111.6) (end 181.1 113.2) (width 0.508) (layer "F.Cu") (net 1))
 (segment (start 158.3115 123.235) (end 167.3115 123.235) (width 0.508) (layer "F.Cu") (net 1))
 (segment (start 167.3115 123.235) (end 180.265 123.235) (width 0.508) (layer "F.Cu") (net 1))
 (segment (start 156.725 129.65) (end 125.05 129.65) (width 0.508) (layer "F.Cu") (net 1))
 (segment (start 180.265 123.235) (end 180.625 122.875) (width 0.508) (layer "F.Cu") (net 1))
 (segment (start 124.315 112.5) (end 125.215 111.6) (width 0.508) (layer "F.Cu") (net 1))
 (via (at 180.625 122.875) (size 0.8) (drill 0.4) (layers "F.Cu" "B.Cu") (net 1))
 (via (at 181.1 113.2) (size 0.8) (drill 0.4) (layers "F.Cu" "B.Cu") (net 1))
 (via (at 181.2 94.5) (size 0.8) (drill 0.4) (layers "F.Cu" "B.Cu") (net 1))
 (via (at 124.625 129.225) (size 0.8) (drill 0.4) (layers "F.Cu" "B.Cu") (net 1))
 (via (at 157.425 128.95) (size 0.8) (drill 0.4) (layers "F.Cu" "B.Cu") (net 1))
 (segment (start 124.315 112.5) (end 124.315 128.915) (width 0.508) (layer "B.Cu") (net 1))
 (segment (start 180.625 122.875) (end 181.1 122.4) (width 0.508) (layer "B.Cu") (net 1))
 (segment (start 181.2 94.5) (end 181.1 94.6) (width 0.508) (layer "B.Cu") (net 1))
 (segment (start 158.3115 128.0635) (end 157.425 128.95) (width 0.508) (layer "B.Cu") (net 1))
 (segment (start 181.1 122.4) (end 181.1 113.2) (width 0.508) (layer "B.Cu") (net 1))
 (segment (start 181.1 94.6) (end 181.1 113.2) (width 0.508) (layer "B.Cu") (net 1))
 (segment (start 124.315 128.915) (end 124.625 129.225) (width 0.508) (layer "B.Cu") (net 1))
 (segment (start 158.3115 123.235) (end 158.3115 128.0635) (width 0.508) (layer "B.Cu") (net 1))
 (segment (start 186 109.9) (end 183.4 109.9) (width 0.25) (layer "F.Cu") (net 4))
 (segment (start 165.8 110) (end 183.1 110) (width 0.25) (layer "F.Cu") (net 4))
 (segment (start 183.4 109.9) (end 183.3 109.8) (width 0.25) (layer "F.Cu") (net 4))
 (segment (start 183.1 110) (end 183.3 109.8) (width 0.25) (layer "F.Cu") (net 4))
 (segment (start 165.8 110) (end 99.2 110) (width 0.25) (layer "F.Cu") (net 4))
 (via (at 183.3 109.8) (size 0.8) (drill 0.4) (layers "F.Cu" "B.Cu") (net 4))
 (via (at 186 109.9) (size 0.8) (drill 0.4) (layers "F.Cu" "B.Cu") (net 4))
 (via (at 99.2 110) (size 0.8) (drill 0.4) (layers "F.Cu" "B.Cu") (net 4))
 (segment (start 186.975 87.21) (end 186.975 108.925) (width 0.25) (layer "B.Cu") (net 4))
 (segment (start 98.915 110.285) (end 99.2 110) (width 0.25) (layer "B.Cu") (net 4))
 (segment (start 183.3 109.8) (end 183.3 102.571) (width 0.25) (layer "B.Cu") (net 4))
 (segment (start 183.3 102.571) (end 184.697 101.174) (width 0.25) (layer "B.Cu") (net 4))
 (segment (start 186.975 108.925) (end 186 109.9) (width 0.25) (layer "B.Cu") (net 4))
 (segment (start 185.83 86.065) (end 186.975 87.21) (width 0.25) (layer "B.Cu") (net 4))
 (segment (start 98.915 112.5) (end 98.915 110.285) (width 0.25) (layer "B.Cu") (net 4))
 (segment (start 175.91 95.99) (end 175.425 96.475) (width 0.25) (layer "F.Cu") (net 21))
 (segment (start 172.8255 114.825) (end 106.8495 114.825) (width 0.25) (layer "F.Cu") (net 21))
 (segment (start 173 114.6505) (end 172.8255 114.825) (width 0.25) (layer "F.Cu") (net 21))
 (segment (start 106.8495 114.825) (end 106.8 114.7755) (width 0.25) (layer "F.Cu") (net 21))
 (segment (start 177.94 95.99) (end 175.91 95.99) (width 0.25) (layer "F.Cu") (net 21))
 (via (at 173 114.6505) (size 0.8) (drill 0.4) (layers "F.Cu" "B.Cu") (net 21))
 (via (at 175.425 96.475) (size 0.8) (drill 0.4) (layers "F.Cu" "B.Cu") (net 21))
 (via (at 106.8 114.7755) (size 0.8) (drill 0.4) (layers "F.Cu" "B.Cu") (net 21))
 (segment (start 175.425 96.475) (end 174.175 97.725) (width 0.25) (layer "B.Cu") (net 21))
 (segment (start 174.175 113.4755) (end 173 114.6505) (width 0.25) (layer "B.Cu") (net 21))
 (segment (start 106.535 114.5105) (end 106.8 114.7755) (width 0.25) (layer "B.Cu") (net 21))
 (segment (start 174.175 97.725) (end 174.175 113.4755) (width 0.25) (layer "B.Cu") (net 21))
 (segment (start 106.535 112.5) (end 106.535 114.5105) (width 0.25) (layer "B.Cu") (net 21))
 (segment (start 104.3 118.65) (end 176.85 118.65) (width 0.25) (layer "F.Cu") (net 24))
 (segment (start 176.85 118.65) (end 177.575 117.925) (width 0.25) (layer "F.Cu") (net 24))
 (via (at 177.575 117.925) (size 0.8) (drill 0.4) (layers "F.Cu" "B.Cu") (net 24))
 (via (at 104.3 118.65) (size 0.8) (drill 0.4) (layers "F.Cu" "B.Cu") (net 24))
 (segment (start 177.94 103.61) (end 177.94 117.56) (width 0.25) (layer "B.Cu") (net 24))
 (segment (start 103.995 118.345) (end 104.3 118.65) (width 0.25) (layer "B.Cu") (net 24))
 (segment (start 103.995 112.5) (end 103.995 118.345) (width 0.25) (layer "B.Cu") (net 24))
 (segment (start 177.94 117.56) (end 177.575 117.925) (width 0.25) (layer "B.Cu") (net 24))
 (segment (start 177.94 101.07) (end 175.566243 101.07) (width 0.25) (layer "F.Cu") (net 23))
 (segment (start 174.49468 116.275) (end 174.72018 116.5005) (width 0.25) (layer "F.Cu") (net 23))
 (segment (start 101.8 116.225) (end 101.85 116.275) (width 0.25) (layer "F.Cu") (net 23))
 (segment (start 101.85 116.275) (end 174.49468 116.275) (width 0.25) (layer "F.Cu") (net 23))
 (segment (start 175.566243 101.07) (end 175.175502 101.460741) (width 0.25) (layer "F.Cu") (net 23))
 (via (at 101.8 116.225) (size 0.8) (drill 0.4) (layers "F.Cu" "B.Cu") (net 23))
 (via (at 174.72018 116.5005) (size 0.8) (drill 0.4) (layers "F.Cu" "B.Cu") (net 23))
 (via (at 175.175502 101.460741) (size 0.8) (drill 0.4) (layers "F.Cu" "B.Cu") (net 23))
 (segment (start 175.175502 101.460741) (end 175.1 101.536243) (width 0.25) (layer "B.Cu") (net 23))
 (segment (start 101.455 112.5) (end 101.455 115.88) (width 0.25) (layer "B.Cu") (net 23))
 (segment (start 175.1 101.536243) (end 175.1 116.12068) (width 0.25) (layer "B.Cu") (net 23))
 (segment (start 101.455 115.88) (end 101.8 116.225) (width 0.25) (layer "B.Cu") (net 23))
 (segment (start 175.1 116.12068) (end 174.72018 116.5005) (width 0.25) (layer "B.Cu") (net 23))
 (segment (start 175.575011 117.900489) (end 89.925489 117.900489) (width 0.25) (layer "F.Cu") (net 22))
 (segment (start 89.925489 117.900489) (end 89.075 117.05) (width 0.25) (layer "F.Cu") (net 22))
 (segment (start 177.77 98.7) (end 177.94 98.53) (width 0.25) (layer "F.Cu") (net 22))
 (segment (start 176.3 98.7) (end 177.77 98.7) (width 0.25) (layer "F.Cu") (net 22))
 (segment (start 175.85 117.6255) (end 175.575011 117.900489) (width 0.25) (layer "F.Cu") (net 22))
 (via (at 89.075 117.05) (size 0.8) (drill 0.4) (layers "F.Cu" "B.Cu") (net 22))
 (via (at 176.3 98.7) (size 0.8) (drill 0.4) (layers "F.Cu" "B.Cu") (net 22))
 (via (at 175.85 117.6255) (size 0.8) (drill 0.4) (layers "F.Cu" "B.Cu") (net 22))
 (segment (start 88.755 112.5) (end 88.755 116.73) (width 0.25) (layer "B.Cu") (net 22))
 (segment (start 176.3 117.1755) (end 175.85 117.6255) (width 0.25) (layer "B.Cu") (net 22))
 (segment (start 176.3 98.7) (end 176.3 117.1755) (width 0.25) (layer "B.Cu") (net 22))
 (segment (start 88.755 116.73) (end 89.075 117.05) (width 0.25) (layer "B.Cu") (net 22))
 (segment (start 182.4 116.7) (end 175.7509 116.7) (width 0.25) (layer "F.Cu") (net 3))
 (segment (start 92 117.225) (end 91.675 116.9) (width 0.25) (layer "F.Cu") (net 3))
 (segment (start 184.697 98.634) (end 183.364032 98.634) (width 0.25) (layer "F.Cu") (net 3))
 (segment (start 175.7509 116.7) (end 175.2259 117.225) (width 0.25) (layer "F.Cu") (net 3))
 (segment (start 183.364032 98.634) (end 182.599016 99.399016) (width 0.25) (layer "F.Cu") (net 3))
 (segment (start 188.4 116.7) (end 182.4 116.7) (width 0.25) (layer "F.Cu") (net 3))
 (segment (start 175.2259 117.225) (end 92 117.225) (width 0.25) (layer "F.Cu") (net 3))
 (via (at 188.4 116.7) (size 0.8) (drill 0.4) (layers "F.Cu" "B.Cu") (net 3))
 (via (at 182.4 116.7) (size 0.8) (drill 0.4) (layers "F.Cu" "B.Cu") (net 3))
 (via (at 91.675 116.9) (size 0.8) (drill 0.4) (layers "F.Cu" "B.Cu") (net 3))
 (via (at 182.599016 99.399016) (size 0.8) (drill 0.4) (layers "F.Cu" "B.Cu") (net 3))
 (segment (start 188.37 86.065) (end 189.1 86.795) (width 0.25) (layer "B.Cu") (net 3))
 (segment (start 91.295 112.5) (end 91.295 116.52) (width 0.25) (layer "B.Cu") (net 3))
 (segment (start 182.4 99.598032) (end 182.599016 99.399016) (width 0.25) (layer "B.Cu") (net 3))
 (segment (start 182.4 116.7) (end 182.4 99.598032) (width 0.25) (layer "B.Cu") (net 3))
 (segment (start 189.1 116) (end 188.4 116.7) (width 0.25) (layer "B.Cu") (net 3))
 (segment (start 189.1 86.795) (end 189.1 116) (width 0.25) (layer "B.Cu") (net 3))
 (segment (start 91.295 116.52) (end 91.675 116.9) (width 0.25) (layer "B.Cu") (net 3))
 (segment (start 117.71 125.335) (end 117.175 124.8) (width 0.25) (layer "F.Cu") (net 25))
 (segment (start 151.195 125.335) (end 117.71 125.335) (width 0.25) (layer "F.Cu") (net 25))
 (via (at 117.175 124.8) (size 0.8) (drill 0.4) (layers "F.Cu" "B.Cu") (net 25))
 (segment (start 116.695 124.32) (end 117.175 124.8) (width 0.25) (layer "B.Cu") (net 25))
 (segment (start 116.695 112.5) (end 116.695 124.32) (width 0.25) (layer "B.Cu") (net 25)))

